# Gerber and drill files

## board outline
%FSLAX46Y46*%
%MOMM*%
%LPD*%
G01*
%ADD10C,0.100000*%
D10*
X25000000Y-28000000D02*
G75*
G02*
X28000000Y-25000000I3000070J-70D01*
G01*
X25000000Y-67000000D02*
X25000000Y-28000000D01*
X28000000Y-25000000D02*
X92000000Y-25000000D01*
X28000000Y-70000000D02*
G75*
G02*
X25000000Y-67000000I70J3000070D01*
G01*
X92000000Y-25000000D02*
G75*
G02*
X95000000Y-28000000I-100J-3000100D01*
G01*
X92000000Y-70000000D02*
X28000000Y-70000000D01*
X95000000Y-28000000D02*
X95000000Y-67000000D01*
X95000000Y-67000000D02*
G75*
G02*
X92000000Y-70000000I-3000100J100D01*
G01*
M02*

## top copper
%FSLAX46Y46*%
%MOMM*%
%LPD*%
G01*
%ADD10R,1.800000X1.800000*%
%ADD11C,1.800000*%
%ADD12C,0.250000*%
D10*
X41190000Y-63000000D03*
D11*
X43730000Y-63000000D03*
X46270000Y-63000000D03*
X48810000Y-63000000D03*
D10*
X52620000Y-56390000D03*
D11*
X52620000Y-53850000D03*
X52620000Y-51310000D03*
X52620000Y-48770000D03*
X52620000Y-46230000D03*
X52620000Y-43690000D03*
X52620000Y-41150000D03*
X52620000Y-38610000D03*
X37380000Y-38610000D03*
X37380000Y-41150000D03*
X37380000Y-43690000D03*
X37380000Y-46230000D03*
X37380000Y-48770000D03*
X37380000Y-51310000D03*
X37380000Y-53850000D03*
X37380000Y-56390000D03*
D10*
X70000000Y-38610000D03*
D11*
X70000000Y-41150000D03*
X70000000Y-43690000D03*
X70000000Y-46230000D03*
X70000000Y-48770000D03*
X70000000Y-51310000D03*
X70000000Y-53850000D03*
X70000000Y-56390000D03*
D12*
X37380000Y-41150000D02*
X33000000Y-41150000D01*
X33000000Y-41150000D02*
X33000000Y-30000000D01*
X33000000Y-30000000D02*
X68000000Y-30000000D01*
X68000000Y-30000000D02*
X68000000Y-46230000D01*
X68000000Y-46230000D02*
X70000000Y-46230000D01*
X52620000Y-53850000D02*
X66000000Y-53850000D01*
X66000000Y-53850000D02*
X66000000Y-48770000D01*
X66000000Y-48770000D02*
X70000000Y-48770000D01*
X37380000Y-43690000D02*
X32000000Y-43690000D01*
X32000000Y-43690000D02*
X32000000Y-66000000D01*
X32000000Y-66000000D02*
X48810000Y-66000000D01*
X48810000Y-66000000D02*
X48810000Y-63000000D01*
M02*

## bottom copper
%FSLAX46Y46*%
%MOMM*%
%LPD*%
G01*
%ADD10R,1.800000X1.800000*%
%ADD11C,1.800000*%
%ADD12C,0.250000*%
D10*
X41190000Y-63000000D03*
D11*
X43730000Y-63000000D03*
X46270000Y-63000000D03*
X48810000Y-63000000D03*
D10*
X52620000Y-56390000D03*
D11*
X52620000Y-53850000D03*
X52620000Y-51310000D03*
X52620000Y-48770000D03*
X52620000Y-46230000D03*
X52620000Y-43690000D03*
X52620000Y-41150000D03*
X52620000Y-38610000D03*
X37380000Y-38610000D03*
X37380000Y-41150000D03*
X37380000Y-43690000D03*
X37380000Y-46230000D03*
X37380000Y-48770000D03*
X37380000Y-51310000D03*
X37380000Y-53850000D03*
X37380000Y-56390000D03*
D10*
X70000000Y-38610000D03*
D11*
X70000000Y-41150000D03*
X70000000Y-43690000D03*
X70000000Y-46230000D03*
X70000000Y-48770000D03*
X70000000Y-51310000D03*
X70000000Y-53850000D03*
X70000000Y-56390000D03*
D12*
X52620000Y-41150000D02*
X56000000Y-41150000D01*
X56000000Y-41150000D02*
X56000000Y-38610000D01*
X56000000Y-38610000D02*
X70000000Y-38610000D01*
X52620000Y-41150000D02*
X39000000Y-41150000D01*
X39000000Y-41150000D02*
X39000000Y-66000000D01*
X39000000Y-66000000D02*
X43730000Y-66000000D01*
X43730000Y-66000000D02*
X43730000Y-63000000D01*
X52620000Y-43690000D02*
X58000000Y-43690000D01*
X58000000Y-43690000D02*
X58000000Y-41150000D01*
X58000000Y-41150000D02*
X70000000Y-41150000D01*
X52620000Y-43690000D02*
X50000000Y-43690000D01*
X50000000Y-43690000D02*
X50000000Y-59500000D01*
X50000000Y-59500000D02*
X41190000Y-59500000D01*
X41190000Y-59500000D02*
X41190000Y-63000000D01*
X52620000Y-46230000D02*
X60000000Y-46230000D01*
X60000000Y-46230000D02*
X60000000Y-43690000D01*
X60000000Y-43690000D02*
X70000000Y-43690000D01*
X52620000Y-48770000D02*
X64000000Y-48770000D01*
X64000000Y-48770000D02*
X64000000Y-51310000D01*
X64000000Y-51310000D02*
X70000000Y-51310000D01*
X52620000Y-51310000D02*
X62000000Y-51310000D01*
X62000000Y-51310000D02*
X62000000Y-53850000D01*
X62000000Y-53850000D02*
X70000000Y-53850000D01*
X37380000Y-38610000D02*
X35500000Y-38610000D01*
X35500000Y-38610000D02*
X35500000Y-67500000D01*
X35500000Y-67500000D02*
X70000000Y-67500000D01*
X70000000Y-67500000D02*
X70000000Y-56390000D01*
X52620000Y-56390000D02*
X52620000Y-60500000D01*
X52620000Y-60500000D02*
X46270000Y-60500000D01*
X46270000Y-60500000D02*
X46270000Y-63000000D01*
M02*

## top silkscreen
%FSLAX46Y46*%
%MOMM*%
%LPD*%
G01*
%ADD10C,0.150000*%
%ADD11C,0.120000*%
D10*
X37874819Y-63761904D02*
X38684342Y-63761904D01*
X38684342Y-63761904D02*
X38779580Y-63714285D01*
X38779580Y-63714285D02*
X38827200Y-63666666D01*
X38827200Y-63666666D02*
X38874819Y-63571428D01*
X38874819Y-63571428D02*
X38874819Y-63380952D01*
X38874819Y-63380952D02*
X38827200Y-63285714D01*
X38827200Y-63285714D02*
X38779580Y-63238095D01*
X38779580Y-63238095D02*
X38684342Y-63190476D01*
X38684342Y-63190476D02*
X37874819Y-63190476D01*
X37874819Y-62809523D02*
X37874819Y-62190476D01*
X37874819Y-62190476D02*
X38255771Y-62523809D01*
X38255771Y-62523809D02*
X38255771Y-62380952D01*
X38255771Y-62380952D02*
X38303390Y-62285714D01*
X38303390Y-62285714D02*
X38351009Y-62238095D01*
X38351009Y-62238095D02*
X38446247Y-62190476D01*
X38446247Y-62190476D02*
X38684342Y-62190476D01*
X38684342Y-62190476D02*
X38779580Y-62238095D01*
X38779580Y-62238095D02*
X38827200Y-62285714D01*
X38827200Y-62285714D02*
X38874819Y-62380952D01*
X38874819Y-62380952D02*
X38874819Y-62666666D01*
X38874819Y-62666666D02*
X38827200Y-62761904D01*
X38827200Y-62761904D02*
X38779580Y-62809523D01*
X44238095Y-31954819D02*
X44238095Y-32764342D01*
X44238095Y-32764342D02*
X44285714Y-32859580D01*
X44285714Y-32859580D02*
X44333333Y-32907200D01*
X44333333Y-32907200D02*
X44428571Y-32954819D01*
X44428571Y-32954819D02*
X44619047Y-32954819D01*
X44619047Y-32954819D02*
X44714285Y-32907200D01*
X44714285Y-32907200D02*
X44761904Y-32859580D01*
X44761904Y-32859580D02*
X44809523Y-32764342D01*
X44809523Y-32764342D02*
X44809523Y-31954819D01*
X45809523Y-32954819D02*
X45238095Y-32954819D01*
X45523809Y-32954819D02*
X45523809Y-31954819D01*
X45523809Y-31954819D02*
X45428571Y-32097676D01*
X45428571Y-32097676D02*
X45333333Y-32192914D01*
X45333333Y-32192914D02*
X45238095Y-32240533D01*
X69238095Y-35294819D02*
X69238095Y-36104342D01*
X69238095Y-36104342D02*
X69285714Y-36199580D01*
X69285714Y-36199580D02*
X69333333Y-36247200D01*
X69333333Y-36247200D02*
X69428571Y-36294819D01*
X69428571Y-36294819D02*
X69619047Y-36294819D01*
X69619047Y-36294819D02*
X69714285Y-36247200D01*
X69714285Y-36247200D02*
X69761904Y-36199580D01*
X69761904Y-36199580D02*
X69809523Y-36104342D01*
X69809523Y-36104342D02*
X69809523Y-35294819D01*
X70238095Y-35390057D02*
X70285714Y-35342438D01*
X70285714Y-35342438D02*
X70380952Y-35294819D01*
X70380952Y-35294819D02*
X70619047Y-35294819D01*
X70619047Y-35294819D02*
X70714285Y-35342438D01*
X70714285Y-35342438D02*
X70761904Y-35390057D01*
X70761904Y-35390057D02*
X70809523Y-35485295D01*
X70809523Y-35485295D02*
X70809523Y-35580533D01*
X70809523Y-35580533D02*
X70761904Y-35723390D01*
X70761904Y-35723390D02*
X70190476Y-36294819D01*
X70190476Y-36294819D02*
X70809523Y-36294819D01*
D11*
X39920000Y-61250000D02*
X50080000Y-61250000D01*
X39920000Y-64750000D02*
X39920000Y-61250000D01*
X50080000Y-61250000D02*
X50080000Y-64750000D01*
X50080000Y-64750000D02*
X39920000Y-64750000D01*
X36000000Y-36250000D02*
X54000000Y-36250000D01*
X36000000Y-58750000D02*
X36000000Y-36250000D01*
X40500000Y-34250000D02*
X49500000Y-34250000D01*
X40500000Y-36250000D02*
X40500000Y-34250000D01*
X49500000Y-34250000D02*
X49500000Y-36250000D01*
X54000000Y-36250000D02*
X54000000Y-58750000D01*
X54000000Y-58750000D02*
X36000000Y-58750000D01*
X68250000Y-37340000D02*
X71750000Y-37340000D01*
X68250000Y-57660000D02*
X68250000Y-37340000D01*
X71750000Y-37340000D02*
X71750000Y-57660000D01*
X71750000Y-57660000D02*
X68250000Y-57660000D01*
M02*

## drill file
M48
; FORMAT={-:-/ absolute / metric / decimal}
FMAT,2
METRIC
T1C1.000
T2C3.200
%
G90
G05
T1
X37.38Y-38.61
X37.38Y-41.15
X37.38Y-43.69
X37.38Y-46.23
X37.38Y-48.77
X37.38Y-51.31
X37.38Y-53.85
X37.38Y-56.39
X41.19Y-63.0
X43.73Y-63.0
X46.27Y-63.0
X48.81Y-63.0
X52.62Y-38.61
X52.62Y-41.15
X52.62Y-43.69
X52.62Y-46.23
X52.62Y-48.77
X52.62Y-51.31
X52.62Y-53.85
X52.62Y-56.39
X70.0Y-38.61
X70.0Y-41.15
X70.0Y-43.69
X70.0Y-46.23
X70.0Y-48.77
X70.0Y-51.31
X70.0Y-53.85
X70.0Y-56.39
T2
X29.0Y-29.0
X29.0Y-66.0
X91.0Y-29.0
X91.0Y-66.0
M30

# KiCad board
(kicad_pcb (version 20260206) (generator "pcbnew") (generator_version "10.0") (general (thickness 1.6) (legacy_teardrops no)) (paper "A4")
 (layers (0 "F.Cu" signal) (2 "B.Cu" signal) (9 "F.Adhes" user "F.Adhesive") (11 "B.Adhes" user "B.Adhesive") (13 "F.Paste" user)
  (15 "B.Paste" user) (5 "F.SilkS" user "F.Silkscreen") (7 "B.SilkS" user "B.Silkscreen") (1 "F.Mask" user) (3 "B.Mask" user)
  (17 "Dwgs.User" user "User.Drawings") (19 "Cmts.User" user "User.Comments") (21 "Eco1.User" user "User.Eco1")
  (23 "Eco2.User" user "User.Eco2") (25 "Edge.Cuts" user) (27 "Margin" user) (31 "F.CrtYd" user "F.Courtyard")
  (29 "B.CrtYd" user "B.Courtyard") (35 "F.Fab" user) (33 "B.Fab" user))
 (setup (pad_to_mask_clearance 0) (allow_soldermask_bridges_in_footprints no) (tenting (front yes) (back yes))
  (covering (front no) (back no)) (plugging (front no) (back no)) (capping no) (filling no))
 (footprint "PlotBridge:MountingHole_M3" (layer "F.Cu") (at 91 66)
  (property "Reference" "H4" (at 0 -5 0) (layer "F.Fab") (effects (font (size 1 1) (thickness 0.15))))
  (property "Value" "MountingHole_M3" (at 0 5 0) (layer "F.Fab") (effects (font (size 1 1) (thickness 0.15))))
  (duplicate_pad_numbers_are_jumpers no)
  (pad "" np_thru_hole circle (at 0 0) (size 3.2 3.2) (drill 3.2) (layers "*.Cu" "*.Mask")))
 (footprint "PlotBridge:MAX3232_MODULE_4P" (layer "F.Cu") (at 45 63 90)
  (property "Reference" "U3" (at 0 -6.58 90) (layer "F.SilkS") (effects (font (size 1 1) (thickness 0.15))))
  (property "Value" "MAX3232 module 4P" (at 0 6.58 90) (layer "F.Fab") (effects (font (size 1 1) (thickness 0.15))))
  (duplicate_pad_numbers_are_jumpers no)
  (fp_line (start 1.75 -5.08) (end 1.75 5.08) (stroke (width 0.12) (type solid)) (layer "F.SilkS"))
  (fp_line (start -1.75 -5.08) (end 1.75 -5.08) (stroke (width 0.12) (type solid)) (layer "F.SilkS"))
  (fp_line (start 1.75 5.08) (end -1.75 5.08) (stroke (width 0.12) (type solid)) (layer "F.SilkS"))
  (fp_line (start -1.75 5.08) (end -1.75 -5.08) (stroke (width 0.12) (type solid)) (layer "F.SilkS"))
  (pad "1" thru_hole rect (at 0 -3.81 90) (size 1.8 1.8) (drill 1) (layers "*.Cu" "*.Mask") (remove_unused_layers no) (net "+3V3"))
  (pad "2" thru_hole circle (at 0 -1.27 90) (size 1.8 1.8) (drill 1) (layers "*.Cu" "*.Mask") (remove_unused_layers no) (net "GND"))
  (pad "3" thru_hole circle (at 0 1.27 90) (size 1.8 1.8) (drill 1) (layers "*.Cu" "*.Mask") (remove_unused_layers no) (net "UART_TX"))
  (pad "4" thru_hole circle (at 0 3.81 90) (size 1.8 1.8) (drill 1) (layers "*.Cu" "*.Mask") (remove_unused_layers no) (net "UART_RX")))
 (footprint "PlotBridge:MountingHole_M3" (layer "F.Cu") (at 91 29)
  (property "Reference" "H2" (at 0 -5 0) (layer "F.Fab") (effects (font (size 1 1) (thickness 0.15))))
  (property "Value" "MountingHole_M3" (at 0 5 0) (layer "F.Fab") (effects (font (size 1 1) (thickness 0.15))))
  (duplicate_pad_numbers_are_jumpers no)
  (pad "" np_thru_hole circle (at 0 0) (size 3.2 3.2) (drill 3.2) (layers "*.Cu" "*.Mask")))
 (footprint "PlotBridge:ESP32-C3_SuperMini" (layer "F.Cu") (at 45 47.5)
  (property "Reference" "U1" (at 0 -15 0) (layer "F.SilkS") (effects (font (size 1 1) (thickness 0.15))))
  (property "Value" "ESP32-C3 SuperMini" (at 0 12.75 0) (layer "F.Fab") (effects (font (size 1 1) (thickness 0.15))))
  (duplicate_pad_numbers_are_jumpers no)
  (fp_line (start -9 -11.25) (end 9 -11.25) (stroke (width 0.12) (type solid)) (layer "F.SilkS"))
  (fp_line (start -9 11.25) (end -9 -11.25) (stroke (width 0.12) (type solid)) (layer "F.SilkS"))
  (fp_line (start -4.5 -13.25) (end 4.5 -13.25) (stroke (width 0.12) (type solid)) (layer "F.SilkS"))
  (fp_line (start -4.5 -11.25) (end -4.5 -13.25) (stroke (width 0.12) (type solid)) (layer "F.SilkS"))
  (fp_line (start 4.5 -13.25) (end 4.5 -11.25) (stroke (width 0.12) (type solid)) (layer "F.SilkS"))
  (fp_line (start 9 -11.25) (end 9 11.25) (stroke (width 0.12) (type solid)) (layer "F.SilkS"))
  (fp_line (start 9 11.25) (end -9 11.25) (stroke (width 0.12) (type solid)) (layer "F.SilkS"))
  (pad "1" thru_hole rect (at 7.62 8.89) (size 1.8 1.8) (drill 1) (layers "*.Cu" "*.Mask") (remove_unused_layers no) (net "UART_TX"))
  (pad "2" thru_hole circle (at 7.62 6.35) (size 1.8 1.8) (drill 1) (layers "*.Cu" "*.Mask") (remove_unused_layers no) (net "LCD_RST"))
  (pad "3" thru_hole circle (at 7.62 3.81) (size 1.8 1.8) (drill 1) (layers "*.Cu" "*.Mask") (remove_unused_layers no) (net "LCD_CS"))
  (pad "4" thru_hole circle (at 7.62 1.27) (size 1.8 1.8) (drill 1) (layers "*.Cu" "*.Mask") (remove_unused_layers no) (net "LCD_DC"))
  (pad "5" thru_hole circle (at 7.62 -1.27) (size 1.8 1.8) (drill 1) (layers "*.Cu" "*.Mask") (remove_unused_layers no) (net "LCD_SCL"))
  (pad "6" thru_hole circle (at 7.62 -3.81) (size 1.8 1.8) (drill 1) (layers "*.Cu" "*.Mask") (remove_unused_layers no) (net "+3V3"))
  (pad "7" thru_hole circle (at 7.62 -6.35) (size 1.8 1.8) (drill 1) (layers "*.Cu" "*.Mask") (remove_unused_layers no) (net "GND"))
  (pad "8" thru_hole circle (at 7.62 -8.89) (size 1.8 1.8) (drill 1) (layers "*.Cu" "*.Mask") (remove_unused_layers no))
  (pad "9" thru_hole circle (at -7.62 -8.89) (size 1.8 1.8) (drill 1) (layers "*.Cu" "*.Mask") (remove_unused_layers no) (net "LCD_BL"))
  (pad "10" thru_hole circle (at -7.62 -6.35) (size 1.8 1.8) (drill 1) (layers "*.Cu" "*.Mask") (remove_unused_layers no) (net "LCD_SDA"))
  (pad "11" thru_hole circle (at -7.62 -3.81) (size 1.8 1.8) (drill 1) (layers "*.Cu" "*.Mask") (remove_unused_layers no) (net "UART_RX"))
  (pad "12" thru_hole circle (at -7.62 -1.27) (size 1.8 1.8) (drill 1) (layers "*.Cu" "*.Mask") (remove_unused_layers no))
  (pad "13" thru_hole circle (at -7.62 1.27) (size 1.8 1.8) (drill 1) (layers "*.Cu" "*.Mask") (remove_unused_layers no))
  (pad "14" thru_hole circle (at -7.62 3.81) (size 1.8 1.8) (drill 1) (layers "*.Cu" "*.Mask") (remove_unused_layers no))
  (pad "15" thru_hole circle (at -7.62 6.35) (size 1.8 1.8) (drill 1) (layers "*.Cu" "*.Mask") (remove_unused_layers no))
  (pad "16" thru_hole circle (at -7.62 8.89) (size 1.8 1.8) (drill 1) (layers "*.Cu" "*.Mask") (remove_unused_layers no)))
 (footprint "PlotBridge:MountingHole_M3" (layer "F.Cu") (at 29 29)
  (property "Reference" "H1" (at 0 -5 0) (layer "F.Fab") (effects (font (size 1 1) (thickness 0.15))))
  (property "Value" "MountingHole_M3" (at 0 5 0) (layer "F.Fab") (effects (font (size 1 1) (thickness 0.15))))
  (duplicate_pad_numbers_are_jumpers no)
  (pad "" np_thru_hole circle (at 0 0) (size 3.2 3.2) (drill 3.2) (layers "*.Cu" "*.Mask")))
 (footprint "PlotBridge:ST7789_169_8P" (layer "F.Cu") (at 70 47.5)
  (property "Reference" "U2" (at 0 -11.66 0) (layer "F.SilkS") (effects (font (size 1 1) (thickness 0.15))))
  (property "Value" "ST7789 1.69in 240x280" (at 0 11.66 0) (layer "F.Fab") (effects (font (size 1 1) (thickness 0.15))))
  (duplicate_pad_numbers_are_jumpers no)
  (fp_line (start -1.75 -10.16) (end 1.75 -10.16) (stroke (width 0.12) (type solid)) (layer "F.SilkS"))
  (fp_line (start -1.75 10.16) (end -1.75 -10.16) (stroke (width 0.12) (type solid)) (layer "F.SilkS"))
  (fp_line (start 1.75 -10.16) (end 1.75 10.16) (stroke (width 0.12) (type solid)) (layer "F.SilkS"))
  (fp_line (start 1.75 10.16) (end -1.75 10.16) (stroke (width 0.12) (type solid)) (layer "F.SilkS"))
  (pad "1" thru_hole rect (at 0 -8.89) (size 1.8 1.8) (drill 1) (layers "*.Cu" "*.Mask") (remove_unused_layers no) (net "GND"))
  (pad "2" thru_hole circle (at 0 -6.35) (size 1.8 1.8) (drill 1) (layers "*.Cu" "*.Mask") (remove_unused_layers no) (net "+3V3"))
  (pad "3" thru_hole circle (at 0 -3.81) (size 1.8 1.8) (drill 1) (layers "*.Cu" "*.Mask") (remove_unused_layers no) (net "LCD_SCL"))
  (pad "4" thru_hole circle (at 0 -1.27) (size 1.8 1.8) (drill 1) (layers "*.Cu" "*.Mask") (remove_unused_layers no) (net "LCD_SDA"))
  (pad "5" thru_hole circle (at 0 1.27) (size 1.8 1.8) (drill 1) (layers "*.Cu" "*.Mask") (remove_unused_layers no) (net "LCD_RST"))
  (pad "6" thru_hole circle (at 0 3.81) (size 1.8 1.8) (drill 1) (layers "*.Cu" "*.Mask") (remove_unused_layers no) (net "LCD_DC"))
  (pad "7" thru_hole circle (at 0 6.35) (size 1.8 1.8) (drill 1) (layers "*.Cu" "*.Mask") (remove_unused_layers no) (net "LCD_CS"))
  (pad "8" thru_hole circle (at 0 8.89) (size 1.8 1.8) (drill 1) (layers "*.Cu" "*.Mask") (remove_unused_layers no) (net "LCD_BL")))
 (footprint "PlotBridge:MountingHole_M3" (layer "F.Cu") (at 29 66)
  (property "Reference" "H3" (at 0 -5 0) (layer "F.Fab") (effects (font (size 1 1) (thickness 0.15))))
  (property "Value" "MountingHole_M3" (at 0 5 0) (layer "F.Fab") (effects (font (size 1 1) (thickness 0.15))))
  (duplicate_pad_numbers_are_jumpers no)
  (pad "" np_thru_hole circle (at 0 0) (size 3.2 3.2) (drill 3.2) (layers "*.Cu" "*.Mask")))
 (gr_arc (start 25 28) (mid 25.8787 25.8787) (end 28 25) (stroke (width 0.1) (type solid)) (layer "Edge.Cuts"))
 (gr_line (start 25 67) (end 25 28) (stroke (width 0.1) (type solid)) (layer "Edge.Cuts"))
 (gr_line (start 28 25) (end 92 25) (stroke (width 0.1) (type solid)) (layer "Edge.Cuts"))
 (gr_arc (start 28 70) (mid 25.8787 69.1213) (end 25 67) (stroke (width 0.1) (type solid)) (layer "Edge.Cuts"))
 (gr_arc (start 92 25) (mid 94.1213 25.8787) (end 95 28) (stroke (width 0.1) (type solid)) (layer "Edge.Cuts"))
 (gr_line (start 92 70) (end 28 70) (stroke (width 0.1) (type solid)) (layer "Edge.Cuts"))
 (gr_line (start 95 28) (end 95 67) (stroke (width 0.1) (type solid)) (layer "Edge.Cuts"))
 (gr_arc (start 95 67) (mid 94.1213 69.1213) (end 92 70) (stroke (width 0.1) (type solid)) (layer "Edge.Cuts"))
 (segment (start 52.62 41.15) (end 56 41.15) (width 0.25) (layer "B.Cu") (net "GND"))
 (segment (start 56 41.15) (end 56 38.61) (width 0.25) (layer "B.Cu") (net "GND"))
 (segment (start 56 38.61) (end 70 38.61) (width 0.25) (layer "B.Cu") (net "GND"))
 (segment (start 52.62 41.15) (end 39 41.15) (width 0.25) (layer "B.Cu") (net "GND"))
 (segment (start 39 41.15) (end 39 66) (width 0.25) (layer "B.Cu") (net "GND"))
 (segment (start 39 66) (end 43.73 66) (width 0.25) (layer "B.Cu") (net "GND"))
 (segment (start 43.73 66) (end 43.73 63) (width 0.25) (layer "B.Cu") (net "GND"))
 (segment (start 52.62 43.69) (end 58 43.69) (width 0.25) (layer "B.Cu") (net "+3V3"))
 (segment (start 58 43.69) (end 58 41.15) (width 0.25) (layer "B.Cu") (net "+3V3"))
 (segment (start 58 41.15) (end 70 41.15) (width 0.25) (layer "B.Cu") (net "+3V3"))
 (segment (start 52.62 43.69) (end 50 43.69) (width 0.25) (layer "B.Cu") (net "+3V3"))
 (segment (start 50 43.69) (end 50 59.5) (width 0.25) (layer "B.Cu") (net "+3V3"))
 (segment (start 50 59.5) (end 41.19 59.5) (width 0.25) (layer "B.Cu") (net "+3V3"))
 (segment (start 41.19 59.5) (end 41.19 63) (width 0.25) (layer "B.Cu") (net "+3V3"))
 (segment (start 52.62 46.23) (end 60 46.23) (width 0.25) (layer "B.Cu") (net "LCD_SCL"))
 (segment (start 60 46.23) (end 60 43.69) (width 0.25) (layer "B.Cu") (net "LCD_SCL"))
 (segment (start 60 43.69) (end 70 43.69) (width 0.25) (layer "B.Cu") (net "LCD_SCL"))
 (segment (start 37.38 41.15) (end 33 41.15) (width 0.25) (layer "F.Cu") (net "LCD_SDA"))
 (segment (start 33 41.15) (end 33 30) (width 0.25) (layer "F.Cu") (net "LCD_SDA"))
 (segment (start 33 30) (end 68 30) (width 0.25) (layer "F.Cu") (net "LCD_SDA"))
 (segment (start 68 30) (end 68 46.23) (width 0.25) (layer "F.Cu") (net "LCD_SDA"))
 (segment (start 68 46.23) (end 70 46.23) (width 0.25) (layer "F.Cu") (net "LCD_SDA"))
 (segment (start 52.62 53.85) (end 66 53.85) (width 0.25) (layer "F.Cu") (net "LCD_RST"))
 (segment (start 66 53.85) (end 66 48.77) (width 0.25) (layer "F.Cu") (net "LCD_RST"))
 (segment (start 66 48.77) (end 70 48.77) (width 0.25) (layer "F.Cu") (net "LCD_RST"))
 (segment (start 52.62 48.77) (end 64 48.77) (width 0.25) (layer "B.Cu") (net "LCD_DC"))
 (segment (start 64 48.77) (end 64 51.31) (width 0.25) (layer "B.Cu") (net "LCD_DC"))
 (segment (start 64 51.31) (end 70 51.31) (width 0.25) (layer "B.Cu") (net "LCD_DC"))
 (segment (start 52.62 51.31) (end 62 51.31) (width 0.25) (layer "B.Cu") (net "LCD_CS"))
 (segment (start 62 51.31) (end 62 53.85) (width 0.25) (layer "B.Cu") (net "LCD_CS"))
 (segment (start 62 53.85) (end 70 53.85) (width 0.25) (layer "B.Cu") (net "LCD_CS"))
 (segment (start 37.38 38.61) (end 35.5 38.61) (width 0.25) (layer "B.Cu") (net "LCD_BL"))
 (segment (start 35.5 38.61) (end 35.5 67.5) (width 0.25) (layer "B.Cu") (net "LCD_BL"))
 (segment (start 35.5 67.5) (end 70 67.5) (width 0.25) (layer "B.Cu") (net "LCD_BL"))
 (segment (start 70 67.5) (end 70 56.39) (width 0.25) (layer "B.Cu") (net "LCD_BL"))
 (segment (start 52.62 56.39) (end 52.62 60.5) (width 0.25) (layer "B.Cu") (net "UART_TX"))
 (segment (start 52.62 60.5) (end 46.27 60.5) (width 0.25) (layer "B.Cu") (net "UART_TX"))
 (segment (start 46.27 60.5) (end 46.27 63) (width 0.25) (layer "B.Cu") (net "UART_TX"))
 (segment (start 37.38 43.69) (end 32 43.69) (width 0.25) (layer "F.Cu") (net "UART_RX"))
 (segment (start 32 43.69) (end 32 66) (width 0.25) (layer "F.Cu") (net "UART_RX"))
 (segment (start 32 66) (end 48.81 66) (width 0.25) (layer "F.Cu") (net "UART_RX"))
 (segment (start 48.81 66) (end 48.81 63) (width 0.25) (layer "F.Cu") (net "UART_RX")))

